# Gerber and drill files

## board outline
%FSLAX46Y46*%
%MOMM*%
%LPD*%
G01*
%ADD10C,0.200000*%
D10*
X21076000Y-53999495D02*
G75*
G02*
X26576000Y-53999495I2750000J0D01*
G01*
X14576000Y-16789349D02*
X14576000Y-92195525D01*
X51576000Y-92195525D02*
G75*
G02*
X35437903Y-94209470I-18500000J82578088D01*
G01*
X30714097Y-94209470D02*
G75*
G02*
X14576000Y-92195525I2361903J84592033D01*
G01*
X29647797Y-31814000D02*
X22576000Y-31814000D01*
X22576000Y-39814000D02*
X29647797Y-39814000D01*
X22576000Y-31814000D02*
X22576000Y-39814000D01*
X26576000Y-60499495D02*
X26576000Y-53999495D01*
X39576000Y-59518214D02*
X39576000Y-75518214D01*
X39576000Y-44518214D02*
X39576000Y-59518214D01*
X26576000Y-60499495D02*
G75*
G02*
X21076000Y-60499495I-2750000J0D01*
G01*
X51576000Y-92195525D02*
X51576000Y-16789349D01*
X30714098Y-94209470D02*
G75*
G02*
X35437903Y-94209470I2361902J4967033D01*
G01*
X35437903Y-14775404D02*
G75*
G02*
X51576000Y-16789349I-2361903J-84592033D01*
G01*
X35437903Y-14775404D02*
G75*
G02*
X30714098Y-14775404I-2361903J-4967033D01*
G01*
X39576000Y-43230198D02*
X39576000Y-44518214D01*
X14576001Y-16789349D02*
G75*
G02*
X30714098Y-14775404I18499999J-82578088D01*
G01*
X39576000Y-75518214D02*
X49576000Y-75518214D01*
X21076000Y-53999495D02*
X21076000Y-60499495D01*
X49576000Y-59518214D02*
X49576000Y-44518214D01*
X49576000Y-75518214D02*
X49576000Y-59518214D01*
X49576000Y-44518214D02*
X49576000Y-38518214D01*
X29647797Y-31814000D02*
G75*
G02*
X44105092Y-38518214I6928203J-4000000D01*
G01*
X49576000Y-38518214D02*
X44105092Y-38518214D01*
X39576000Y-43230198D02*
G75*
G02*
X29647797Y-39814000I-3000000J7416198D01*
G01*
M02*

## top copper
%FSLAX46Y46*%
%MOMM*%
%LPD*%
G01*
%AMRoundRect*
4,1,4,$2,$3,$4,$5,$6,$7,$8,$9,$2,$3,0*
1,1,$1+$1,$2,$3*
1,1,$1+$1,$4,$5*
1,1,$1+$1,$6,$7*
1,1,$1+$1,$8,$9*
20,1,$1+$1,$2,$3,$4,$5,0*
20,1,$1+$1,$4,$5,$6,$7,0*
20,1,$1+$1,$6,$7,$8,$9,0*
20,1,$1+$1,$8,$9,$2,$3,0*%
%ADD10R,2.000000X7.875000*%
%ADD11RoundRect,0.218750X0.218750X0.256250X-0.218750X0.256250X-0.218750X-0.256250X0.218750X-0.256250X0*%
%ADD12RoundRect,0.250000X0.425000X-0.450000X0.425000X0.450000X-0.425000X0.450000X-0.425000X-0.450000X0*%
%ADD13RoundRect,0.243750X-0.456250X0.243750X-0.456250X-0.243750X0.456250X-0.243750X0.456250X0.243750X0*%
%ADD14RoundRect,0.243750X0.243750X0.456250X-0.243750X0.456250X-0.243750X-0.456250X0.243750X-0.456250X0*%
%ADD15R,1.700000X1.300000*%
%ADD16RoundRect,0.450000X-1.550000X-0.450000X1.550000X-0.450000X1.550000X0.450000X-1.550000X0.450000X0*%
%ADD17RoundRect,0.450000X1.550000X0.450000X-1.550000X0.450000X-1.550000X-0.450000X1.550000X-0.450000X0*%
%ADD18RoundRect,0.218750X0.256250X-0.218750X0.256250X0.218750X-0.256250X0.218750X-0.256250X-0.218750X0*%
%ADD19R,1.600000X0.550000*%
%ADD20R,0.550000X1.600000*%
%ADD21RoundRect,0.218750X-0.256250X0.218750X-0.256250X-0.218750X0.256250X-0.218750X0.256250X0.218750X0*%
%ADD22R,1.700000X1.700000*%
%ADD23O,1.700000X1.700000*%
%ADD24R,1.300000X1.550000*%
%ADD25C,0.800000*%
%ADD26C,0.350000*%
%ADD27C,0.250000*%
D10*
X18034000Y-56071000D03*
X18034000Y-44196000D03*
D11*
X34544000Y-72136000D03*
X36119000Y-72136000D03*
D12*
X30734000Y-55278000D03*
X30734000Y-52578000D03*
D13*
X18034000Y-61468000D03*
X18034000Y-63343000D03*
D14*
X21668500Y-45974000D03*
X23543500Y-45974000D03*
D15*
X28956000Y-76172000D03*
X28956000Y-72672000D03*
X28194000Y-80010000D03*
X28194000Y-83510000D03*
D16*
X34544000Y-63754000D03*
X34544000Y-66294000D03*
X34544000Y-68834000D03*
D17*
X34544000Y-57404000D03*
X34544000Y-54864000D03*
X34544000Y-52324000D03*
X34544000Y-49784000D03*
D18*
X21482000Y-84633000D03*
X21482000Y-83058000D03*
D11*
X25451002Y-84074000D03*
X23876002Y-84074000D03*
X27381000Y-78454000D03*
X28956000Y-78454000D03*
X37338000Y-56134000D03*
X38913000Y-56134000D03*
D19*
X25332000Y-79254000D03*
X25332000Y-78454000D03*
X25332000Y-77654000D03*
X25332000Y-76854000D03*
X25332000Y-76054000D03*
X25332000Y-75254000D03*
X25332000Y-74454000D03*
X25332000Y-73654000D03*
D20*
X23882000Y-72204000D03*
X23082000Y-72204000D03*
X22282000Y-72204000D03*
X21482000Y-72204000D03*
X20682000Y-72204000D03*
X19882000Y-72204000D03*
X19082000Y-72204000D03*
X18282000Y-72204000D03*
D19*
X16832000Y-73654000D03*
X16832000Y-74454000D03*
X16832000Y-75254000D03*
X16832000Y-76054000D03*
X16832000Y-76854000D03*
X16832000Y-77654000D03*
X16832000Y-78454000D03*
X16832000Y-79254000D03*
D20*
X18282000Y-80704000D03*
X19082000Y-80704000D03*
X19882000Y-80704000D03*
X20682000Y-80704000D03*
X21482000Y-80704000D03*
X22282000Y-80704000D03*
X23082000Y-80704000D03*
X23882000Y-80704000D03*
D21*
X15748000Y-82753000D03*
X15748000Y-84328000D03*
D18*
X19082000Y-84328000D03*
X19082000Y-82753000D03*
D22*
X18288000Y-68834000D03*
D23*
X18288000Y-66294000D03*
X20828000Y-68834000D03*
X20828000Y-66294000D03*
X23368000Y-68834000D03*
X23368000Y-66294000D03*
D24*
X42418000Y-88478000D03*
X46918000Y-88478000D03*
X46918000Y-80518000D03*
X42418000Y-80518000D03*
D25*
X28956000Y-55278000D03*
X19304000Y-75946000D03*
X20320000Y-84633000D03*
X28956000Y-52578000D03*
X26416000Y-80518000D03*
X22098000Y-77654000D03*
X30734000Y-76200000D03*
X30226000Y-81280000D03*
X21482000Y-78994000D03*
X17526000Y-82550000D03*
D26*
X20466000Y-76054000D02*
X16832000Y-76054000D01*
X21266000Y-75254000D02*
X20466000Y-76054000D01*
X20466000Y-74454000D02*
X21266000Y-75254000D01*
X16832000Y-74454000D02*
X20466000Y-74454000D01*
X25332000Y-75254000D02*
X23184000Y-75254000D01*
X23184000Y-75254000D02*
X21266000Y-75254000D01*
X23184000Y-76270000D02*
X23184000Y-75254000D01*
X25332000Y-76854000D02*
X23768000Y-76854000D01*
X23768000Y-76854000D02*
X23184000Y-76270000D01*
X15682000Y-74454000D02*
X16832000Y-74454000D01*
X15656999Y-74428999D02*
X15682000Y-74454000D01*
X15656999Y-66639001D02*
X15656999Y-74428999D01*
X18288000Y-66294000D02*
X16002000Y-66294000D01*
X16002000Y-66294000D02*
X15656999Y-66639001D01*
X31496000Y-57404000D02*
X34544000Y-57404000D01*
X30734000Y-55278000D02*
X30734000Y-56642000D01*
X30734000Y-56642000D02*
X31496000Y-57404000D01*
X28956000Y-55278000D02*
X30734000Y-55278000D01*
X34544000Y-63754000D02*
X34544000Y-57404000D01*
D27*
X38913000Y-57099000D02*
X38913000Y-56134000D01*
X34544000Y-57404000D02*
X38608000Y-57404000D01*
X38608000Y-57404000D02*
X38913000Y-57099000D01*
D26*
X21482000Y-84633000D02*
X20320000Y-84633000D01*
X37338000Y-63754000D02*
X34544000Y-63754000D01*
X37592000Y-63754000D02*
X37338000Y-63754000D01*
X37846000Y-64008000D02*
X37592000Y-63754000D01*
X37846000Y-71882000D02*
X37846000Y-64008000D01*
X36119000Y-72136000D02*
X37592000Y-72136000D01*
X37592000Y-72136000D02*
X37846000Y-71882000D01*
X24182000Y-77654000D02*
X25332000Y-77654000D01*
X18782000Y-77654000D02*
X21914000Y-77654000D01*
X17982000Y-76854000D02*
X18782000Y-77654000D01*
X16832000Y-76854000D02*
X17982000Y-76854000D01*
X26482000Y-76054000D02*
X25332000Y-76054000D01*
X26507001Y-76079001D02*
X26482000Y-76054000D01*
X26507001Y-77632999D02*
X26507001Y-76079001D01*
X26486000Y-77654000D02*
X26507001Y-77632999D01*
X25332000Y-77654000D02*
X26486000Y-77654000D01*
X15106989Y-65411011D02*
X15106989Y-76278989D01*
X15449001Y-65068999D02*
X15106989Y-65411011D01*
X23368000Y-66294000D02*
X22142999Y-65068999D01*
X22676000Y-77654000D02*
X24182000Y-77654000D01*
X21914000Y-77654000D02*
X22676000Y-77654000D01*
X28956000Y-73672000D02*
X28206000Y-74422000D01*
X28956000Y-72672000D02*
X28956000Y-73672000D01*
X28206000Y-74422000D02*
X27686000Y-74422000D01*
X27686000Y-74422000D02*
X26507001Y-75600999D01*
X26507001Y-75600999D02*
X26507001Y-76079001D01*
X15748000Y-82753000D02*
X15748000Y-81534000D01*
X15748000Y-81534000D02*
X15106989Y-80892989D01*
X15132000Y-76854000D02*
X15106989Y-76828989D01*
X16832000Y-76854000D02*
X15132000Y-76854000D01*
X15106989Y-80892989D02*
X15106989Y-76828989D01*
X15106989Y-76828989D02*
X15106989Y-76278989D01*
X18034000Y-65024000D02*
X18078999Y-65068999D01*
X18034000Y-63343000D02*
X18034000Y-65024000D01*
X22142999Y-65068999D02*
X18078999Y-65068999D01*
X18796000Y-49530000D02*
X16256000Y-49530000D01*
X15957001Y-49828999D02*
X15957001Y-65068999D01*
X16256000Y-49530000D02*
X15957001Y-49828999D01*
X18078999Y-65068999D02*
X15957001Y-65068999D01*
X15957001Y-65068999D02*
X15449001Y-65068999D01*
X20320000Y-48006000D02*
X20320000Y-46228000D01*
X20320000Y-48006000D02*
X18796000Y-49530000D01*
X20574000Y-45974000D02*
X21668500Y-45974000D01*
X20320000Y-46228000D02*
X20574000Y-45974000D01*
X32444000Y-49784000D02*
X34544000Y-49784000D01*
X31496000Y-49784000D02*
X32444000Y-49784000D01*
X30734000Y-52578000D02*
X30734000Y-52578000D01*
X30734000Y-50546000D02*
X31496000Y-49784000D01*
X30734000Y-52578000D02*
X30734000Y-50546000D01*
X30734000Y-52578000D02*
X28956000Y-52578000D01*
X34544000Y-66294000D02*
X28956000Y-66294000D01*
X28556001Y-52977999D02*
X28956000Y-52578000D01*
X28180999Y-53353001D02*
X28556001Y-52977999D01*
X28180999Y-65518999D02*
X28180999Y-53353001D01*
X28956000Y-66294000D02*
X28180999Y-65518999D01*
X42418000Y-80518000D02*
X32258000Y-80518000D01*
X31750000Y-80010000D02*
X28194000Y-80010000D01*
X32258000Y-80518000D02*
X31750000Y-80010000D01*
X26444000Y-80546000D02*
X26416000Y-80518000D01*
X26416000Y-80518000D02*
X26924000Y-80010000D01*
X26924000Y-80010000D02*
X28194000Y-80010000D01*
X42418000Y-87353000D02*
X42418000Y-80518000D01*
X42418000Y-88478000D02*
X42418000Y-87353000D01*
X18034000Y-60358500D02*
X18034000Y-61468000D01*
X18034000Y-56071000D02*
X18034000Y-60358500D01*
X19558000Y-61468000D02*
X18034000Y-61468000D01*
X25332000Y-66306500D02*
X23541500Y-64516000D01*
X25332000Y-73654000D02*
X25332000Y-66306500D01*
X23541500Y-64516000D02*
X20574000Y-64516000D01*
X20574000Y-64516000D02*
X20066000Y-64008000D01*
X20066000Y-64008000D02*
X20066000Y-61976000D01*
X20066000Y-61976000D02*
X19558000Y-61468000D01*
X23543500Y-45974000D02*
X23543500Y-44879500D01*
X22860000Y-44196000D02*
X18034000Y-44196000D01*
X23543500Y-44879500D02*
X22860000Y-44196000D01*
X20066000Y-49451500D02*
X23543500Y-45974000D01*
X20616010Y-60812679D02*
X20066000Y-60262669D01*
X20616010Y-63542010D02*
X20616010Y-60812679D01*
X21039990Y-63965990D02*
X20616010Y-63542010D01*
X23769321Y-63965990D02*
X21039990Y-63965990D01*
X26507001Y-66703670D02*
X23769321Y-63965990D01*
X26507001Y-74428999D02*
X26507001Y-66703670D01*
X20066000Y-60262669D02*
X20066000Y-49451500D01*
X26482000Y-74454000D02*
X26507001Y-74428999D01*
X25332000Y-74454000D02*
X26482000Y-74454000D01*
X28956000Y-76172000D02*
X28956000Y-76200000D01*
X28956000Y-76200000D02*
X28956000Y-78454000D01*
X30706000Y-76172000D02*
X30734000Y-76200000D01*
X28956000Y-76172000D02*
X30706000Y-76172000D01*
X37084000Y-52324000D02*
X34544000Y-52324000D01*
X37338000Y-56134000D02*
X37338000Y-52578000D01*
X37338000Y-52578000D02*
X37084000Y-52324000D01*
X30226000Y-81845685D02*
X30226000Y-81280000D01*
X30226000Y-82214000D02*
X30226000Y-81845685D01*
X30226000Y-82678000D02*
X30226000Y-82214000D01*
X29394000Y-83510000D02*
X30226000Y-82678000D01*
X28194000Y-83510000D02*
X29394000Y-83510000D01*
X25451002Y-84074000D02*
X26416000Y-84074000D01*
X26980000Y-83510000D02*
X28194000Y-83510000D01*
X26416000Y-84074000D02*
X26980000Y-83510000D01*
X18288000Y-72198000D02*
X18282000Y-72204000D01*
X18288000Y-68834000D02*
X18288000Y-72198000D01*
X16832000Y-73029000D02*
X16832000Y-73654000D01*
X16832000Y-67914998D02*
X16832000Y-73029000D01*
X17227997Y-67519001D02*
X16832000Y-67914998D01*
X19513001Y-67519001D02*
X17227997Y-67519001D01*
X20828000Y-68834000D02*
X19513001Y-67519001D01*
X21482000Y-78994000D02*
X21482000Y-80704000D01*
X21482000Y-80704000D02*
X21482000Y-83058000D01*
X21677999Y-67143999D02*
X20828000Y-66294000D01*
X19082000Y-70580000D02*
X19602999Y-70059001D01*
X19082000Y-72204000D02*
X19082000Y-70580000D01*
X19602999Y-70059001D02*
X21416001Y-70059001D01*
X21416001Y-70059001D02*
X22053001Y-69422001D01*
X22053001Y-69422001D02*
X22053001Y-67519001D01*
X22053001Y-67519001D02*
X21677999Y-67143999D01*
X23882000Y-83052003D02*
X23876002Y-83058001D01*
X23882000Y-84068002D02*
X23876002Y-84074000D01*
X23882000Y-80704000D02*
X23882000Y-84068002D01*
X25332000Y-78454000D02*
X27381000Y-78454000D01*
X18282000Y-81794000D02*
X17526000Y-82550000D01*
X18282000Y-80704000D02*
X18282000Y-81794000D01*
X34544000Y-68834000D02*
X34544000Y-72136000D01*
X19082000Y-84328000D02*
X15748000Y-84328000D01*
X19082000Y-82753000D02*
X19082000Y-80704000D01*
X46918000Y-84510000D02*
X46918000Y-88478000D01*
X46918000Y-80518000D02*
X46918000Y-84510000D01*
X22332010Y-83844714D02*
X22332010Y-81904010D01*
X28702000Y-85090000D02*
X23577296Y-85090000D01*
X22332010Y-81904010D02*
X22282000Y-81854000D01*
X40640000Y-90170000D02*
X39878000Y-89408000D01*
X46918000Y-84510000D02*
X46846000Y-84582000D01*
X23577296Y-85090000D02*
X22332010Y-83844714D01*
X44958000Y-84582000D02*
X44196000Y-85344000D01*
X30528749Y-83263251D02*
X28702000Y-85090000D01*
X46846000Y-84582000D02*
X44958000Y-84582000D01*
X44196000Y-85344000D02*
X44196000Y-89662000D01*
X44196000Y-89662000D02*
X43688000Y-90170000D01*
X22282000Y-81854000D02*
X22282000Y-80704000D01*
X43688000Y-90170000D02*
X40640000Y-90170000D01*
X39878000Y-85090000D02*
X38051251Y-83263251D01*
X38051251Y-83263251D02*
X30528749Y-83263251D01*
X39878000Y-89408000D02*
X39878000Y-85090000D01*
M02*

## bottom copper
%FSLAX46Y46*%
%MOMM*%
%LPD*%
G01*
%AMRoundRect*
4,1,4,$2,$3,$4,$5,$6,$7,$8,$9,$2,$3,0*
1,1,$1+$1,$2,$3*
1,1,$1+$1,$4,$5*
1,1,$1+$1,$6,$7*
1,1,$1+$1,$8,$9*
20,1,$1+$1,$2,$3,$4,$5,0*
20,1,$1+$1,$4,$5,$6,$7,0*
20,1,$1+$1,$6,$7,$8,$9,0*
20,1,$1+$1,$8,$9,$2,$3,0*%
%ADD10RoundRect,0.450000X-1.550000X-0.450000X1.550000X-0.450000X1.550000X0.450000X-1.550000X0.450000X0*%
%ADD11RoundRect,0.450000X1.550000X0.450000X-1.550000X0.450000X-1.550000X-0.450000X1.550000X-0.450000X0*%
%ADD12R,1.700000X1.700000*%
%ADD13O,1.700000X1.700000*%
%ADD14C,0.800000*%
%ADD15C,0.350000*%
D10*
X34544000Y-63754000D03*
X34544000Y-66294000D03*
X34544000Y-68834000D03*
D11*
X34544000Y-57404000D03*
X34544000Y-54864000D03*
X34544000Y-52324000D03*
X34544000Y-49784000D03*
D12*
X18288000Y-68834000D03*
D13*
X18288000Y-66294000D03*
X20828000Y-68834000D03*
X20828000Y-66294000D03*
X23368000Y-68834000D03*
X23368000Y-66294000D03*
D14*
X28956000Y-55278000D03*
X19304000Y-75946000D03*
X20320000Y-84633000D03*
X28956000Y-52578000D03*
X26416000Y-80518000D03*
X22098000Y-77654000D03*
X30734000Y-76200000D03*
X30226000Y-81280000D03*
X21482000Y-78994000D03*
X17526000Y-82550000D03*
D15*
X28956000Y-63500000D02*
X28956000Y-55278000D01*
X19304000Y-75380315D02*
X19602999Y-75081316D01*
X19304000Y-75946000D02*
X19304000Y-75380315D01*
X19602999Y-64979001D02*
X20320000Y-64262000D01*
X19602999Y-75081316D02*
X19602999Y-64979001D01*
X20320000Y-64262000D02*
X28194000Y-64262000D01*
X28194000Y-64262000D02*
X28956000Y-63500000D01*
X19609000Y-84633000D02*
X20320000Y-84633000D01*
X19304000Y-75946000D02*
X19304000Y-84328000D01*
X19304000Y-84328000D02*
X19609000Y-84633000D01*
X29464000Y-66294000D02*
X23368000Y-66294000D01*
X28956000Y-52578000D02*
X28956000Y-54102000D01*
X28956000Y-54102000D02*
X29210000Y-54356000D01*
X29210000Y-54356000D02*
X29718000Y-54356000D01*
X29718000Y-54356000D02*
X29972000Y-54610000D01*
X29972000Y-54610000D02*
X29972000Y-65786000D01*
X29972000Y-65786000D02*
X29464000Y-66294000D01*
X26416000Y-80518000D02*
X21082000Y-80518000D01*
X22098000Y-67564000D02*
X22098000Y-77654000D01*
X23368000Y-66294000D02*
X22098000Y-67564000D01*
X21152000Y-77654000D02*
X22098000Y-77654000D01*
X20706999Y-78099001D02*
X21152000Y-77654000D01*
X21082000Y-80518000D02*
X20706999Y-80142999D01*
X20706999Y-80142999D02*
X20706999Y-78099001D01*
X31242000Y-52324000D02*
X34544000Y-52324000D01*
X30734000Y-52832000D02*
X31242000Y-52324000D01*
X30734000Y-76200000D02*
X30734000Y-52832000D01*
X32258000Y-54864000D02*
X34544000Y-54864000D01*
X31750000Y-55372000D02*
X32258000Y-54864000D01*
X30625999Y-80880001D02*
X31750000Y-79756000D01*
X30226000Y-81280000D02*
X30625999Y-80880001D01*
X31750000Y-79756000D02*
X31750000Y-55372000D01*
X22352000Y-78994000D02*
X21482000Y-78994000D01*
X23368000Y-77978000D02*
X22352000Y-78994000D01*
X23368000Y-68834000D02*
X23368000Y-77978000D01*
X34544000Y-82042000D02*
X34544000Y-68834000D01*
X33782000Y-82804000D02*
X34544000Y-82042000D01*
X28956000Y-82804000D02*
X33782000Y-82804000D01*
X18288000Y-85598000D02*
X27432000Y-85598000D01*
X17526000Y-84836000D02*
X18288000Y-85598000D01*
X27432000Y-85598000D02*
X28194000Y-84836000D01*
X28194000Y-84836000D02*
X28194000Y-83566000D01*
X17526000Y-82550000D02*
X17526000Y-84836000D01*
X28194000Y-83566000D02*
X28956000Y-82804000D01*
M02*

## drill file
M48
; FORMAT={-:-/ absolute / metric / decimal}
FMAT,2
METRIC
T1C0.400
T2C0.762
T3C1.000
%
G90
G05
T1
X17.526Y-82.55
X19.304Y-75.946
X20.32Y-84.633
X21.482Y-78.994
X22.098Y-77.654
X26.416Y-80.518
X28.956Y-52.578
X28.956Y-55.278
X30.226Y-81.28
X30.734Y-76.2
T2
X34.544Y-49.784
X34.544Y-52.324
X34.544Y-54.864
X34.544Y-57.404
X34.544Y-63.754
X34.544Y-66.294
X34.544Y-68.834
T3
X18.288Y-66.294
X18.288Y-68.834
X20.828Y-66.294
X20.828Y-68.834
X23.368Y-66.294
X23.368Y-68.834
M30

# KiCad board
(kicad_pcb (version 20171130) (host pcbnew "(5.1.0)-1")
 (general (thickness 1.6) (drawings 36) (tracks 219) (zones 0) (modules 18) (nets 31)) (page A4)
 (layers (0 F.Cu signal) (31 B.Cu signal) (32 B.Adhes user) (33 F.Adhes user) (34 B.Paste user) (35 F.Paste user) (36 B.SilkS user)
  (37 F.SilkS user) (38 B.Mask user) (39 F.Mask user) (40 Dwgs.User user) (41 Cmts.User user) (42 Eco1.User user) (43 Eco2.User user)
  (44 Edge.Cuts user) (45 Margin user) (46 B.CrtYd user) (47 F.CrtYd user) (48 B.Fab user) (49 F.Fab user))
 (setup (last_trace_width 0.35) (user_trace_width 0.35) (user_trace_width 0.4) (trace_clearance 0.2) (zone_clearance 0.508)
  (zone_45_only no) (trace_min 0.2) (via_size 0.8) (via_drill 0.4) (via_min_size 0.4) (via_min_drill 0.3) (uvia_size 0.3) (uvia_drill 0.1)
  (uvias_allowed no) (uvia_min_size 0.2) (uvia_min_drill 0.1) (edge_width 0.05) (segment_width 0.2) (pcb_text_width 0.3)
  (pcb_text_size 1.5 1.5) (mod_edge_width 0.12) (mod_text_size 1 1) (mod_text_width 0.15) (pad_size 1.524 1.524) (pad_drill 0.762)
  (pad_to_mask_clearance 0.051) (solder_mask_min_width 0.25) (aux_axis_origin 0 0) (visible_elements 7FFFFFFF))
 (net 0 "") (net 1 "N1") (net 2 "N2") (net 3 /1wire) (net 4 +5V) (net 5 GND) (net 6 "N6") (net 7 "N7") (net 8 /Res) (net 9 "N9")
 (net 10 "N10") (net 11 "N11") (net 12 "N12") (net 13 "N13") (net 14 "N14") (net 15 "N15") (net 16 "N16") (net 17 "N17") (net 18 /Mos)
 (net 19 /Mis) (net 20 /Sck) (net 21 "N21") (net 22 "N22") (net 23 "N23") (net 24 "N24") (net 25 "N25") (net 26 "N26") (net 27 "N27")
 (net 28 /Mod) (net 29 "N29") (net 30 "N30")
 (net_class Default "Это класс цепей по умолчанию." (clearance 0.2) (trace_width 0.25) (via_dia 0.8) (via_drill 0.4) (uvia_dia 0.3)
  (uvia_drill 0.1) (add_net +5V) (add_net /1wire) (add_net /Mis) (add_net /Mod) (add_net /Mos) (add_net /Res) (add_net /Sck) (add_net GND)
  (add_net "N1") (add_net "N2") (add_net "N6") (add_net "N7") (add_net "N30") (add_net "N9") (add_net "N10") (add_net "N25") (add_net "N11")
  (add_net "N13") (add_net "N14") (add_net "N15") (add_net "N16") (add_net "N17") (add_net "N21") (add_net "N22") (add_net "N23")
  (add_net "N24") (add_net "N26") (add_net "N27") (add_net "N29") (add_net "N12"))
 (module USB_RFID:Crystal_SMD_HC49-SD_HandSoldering (layer F.Cu) (at 18.034 50.1335 90)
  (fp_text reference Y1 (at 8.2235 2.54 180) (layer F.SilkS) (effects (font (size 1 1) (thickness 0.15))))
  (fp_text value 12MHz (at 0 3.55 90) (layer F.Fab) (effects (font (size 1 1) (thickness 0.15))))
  (pad 1 smd rect (at -5.9375 0 90) (size 7.875 2) (layers F.Cu F.Paste F.Mask) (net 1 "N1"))
  (pad 2 smd rect (at 5.9375 0 90) (size 7.875 2) (layers F.Cu F.Paste F.Mask) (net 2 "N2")))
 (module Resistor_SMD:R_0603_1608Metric (layer F.Cu) (at 35.3315 72.136 180)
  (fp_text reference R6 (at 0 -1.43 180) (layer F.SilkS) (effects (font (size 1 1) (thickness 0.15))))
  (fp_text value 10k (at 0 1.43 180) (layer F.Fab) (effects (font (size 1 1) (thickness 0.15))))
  (pad 2 smd roundrect (at 0.7875 0 180) (size 0.875 0.95) (layers F.Cu F.Paste F.Mask) (roundrect_rratio 0.25) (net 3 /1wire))
  (pad 1 smd roundrect (at -0.7875 0 180) (size 0.875 0.95) (layers F.Cu F.Paste F.Mask) (roundrect_rratio 0.25) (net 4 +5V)))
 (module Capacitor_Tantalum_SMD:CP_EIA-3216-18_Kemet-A (layer F.Cu) (at 30.734 53.928 90)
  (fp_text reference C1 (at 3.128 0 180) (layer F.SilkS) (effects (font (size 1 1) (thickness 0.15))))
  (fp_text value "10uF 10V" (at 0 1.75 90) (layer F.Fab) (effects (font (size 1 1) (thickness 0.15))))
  (pad 1 smd roundrect (at -1.35 0 90) (size 1.4 1.35) (layers F.Cu F.Paste F.Mask) (roundrect_rratio 0.185185) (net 4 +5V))
  (pad 2 smd roundrect (at 1.35 0 90) (size 1.4 1.35) (layers F.Cu F.Paste F.Mask) (roundrect_rratio 0.185185) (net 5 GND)))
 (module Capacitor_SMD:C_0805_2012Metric (layer F.Cu) (at 18.034 62.4055 270)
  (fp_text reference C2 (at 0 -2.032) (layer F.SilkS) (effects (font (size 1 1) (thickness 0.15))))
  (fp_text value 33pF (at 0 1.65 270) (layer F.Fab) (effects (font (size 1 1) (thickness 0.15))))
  (pad 1 smd roundrect (at -0.9375 0 270) (size 0.975 1.4) (layers F.Cu F.Paste F.Mask) (roundrect_rratio 0.25) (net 1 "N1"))
  (pad 2 smd roundrect (at 0.9375 0 270) (size 0.975 1.4) (layers F.Cu F.Paste F.Mask) (roundrect_rratio 0.25) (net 5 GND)))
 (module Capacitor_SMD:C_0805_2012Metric (layer F.Cu) (at 22.606 45.974 180)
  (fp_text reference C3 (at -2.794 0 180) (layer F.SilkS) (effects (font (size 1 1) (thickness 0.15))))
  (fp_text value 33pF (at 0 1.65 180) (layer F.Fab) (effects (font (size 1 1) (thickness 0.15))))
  (pad 2 smd roundrect (at 0.9375 0 180) (size 0.975 1.4) (layers F.Cu F.Paste F.Mask) (roundrect_rratio 0.25) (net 5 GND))
  (pad 1 smd roundrect (at -0.9375 0 180) (size 0.975 1.4) (layers F.Cu F.Paste F.Mask) (roundrect_rratio 0.25) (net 2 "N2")))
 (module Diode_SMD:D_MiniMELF (layer F.Cu) (at 28.956 74.422 90)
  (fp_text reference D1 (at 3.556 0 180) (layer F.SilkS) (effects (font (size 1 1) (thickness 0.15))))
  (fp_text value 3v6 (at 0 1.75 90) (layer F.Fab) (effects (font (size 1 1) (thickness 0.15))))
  (pad 1 smd rect (at -1.75 0 90) (size 1.3 1.7) (layers F.Cu F.Paste F.Mask) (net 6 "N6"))
  (pad 2 smd rect (at 1.75 0 90) (size 1.3 1.7) (layers F.Cu F.Paste F.Mask) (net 5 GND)))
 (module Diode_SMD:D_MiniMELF (layer F.Cu) (at 28.194 81.76 90)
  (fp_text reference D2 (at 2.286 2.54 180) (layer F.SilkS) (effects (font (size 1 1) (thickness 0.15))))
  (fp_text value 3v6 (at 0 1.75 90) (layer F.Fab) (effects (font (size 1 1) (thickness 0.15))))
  (pad 2 smd rect (at 1.75 0 90) (size 1.3 1.7) (layers F.Cu F.Paste F.Mask) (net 5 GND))
  (pad 1 smd rect (at -1.75 0 90) (size 1.3 1.7) (layers F.Cu F.Paste F.Mask) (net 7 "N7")))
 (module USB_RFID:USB (layer F.Cu) (at 34.544 61.214)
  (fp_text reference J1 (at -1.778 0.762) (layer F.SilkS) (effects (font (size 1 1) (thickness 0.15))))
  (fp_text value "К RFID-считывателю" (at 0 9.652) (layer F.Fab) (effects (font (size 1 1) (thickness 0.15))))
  (pad 1 thru_hole roundrect (at 0 2.54) (size 4 1.8) (drill 0.762) (layers *.Cu *.Mask) (roundrect_rratio 0.25) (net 4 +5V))
  (pad 2 thru_hole roundrect (at 0 5.08) (size 4 1.8) (drill 0.762) (layers *.Cu *.Mask) (roundrect_rratio 0.25) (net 5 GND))
  (pad 3 thru_hole roundrect (at 0 7.62) (size 4 1.8) (drill 0.762) (layers *.Cu *.Mask) (roundrect_rratio 0.25) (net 3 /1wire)))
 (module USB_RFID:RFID (layer F.Cu) (at 34.544 59.944 180)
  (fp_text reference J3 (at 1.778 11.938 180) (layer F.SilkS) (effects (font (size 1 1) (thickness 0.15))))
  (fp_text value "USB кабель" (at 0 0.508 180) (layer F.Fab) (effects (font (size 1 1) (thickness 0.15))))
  (pad 1 thru_hole roundrect (at 0 2.54 180) (size 4 1.8) (drill 0.762) (layers *.Cu *.Mask) (roundrect_rratio 0.25) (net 4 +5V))
  (pad 2 thru_hole roundrect (at 0 5.08 180) (size 4 1.8) (drill 0.762) (layers *.Cu *.Mask) (roundrect_rratio 0.25) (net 7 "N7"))
  (pad 3 thru_hole roundrect (at 0 7.62 180) (size 4 1.8) (drill 0.762) (layers *.Cu *.Mask) (roundrect_rratio 0.25) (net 6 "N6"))
  (pad 4 thru_hole roundrect (at 0 10.16 180) (size 4 1.8) (drill 0.762) (layers *.Cu *.Mask) (roundrect_rratio 0.25) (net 5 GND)))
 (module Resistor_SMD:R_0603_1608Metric (layer F.Cu) (at 21.482 83.8455 90)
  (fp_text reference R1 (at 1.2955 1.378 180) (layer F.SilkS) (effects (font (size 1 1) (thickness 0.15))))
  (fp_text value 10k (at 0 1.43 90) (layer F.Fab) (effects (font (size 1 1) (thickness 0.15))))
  (pad 1 smd roundrect (at -0.7875 0 90) (size 0.875 0.95) (layers F.Cu F.Paste F.Mask) (roundrect_rratio 0.25) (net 4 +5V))
  (pad 2 smd roundrect (at 0.7875 0 90) (size 0.875 0.95) (layers F.Cu F.Paste F.Mask) (roundrect_rratio 0.25) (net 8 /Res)))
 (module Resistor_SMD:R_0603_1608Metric (layer F.Cu) (at 24.663502 84.074 180)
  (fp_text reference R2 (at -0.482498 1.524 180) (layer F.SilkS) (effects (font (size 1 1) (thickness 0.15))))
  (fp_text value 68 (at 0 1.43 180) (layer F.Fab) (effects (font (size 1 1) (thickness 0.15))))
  (pad 1 smd roundrect (at -0.7875 0 180) (size 0.875 0.95) (layers F.Cu F.Paste F.Mask) (roundrect_rratio 0.25) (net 7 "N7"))
  (pad 2 smd roundrect (at 0.7875 0 180) (size 0.875 0.95) (layers F.Cu F.Paste F.Mask) (roundrect_rratio 0.25) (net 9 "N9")))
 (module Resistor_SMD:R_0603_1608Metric (layer F.Cu) (at 28.1685 78.454 180)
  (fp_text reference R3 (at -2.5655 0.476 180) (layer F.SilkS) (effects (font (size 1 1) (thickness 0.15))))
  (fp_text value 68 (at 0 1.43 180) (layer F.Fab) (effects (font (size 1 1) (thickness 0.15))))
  (pad 2 smd roundrect (at 0.7875 0 180) (size 0.875 0.95) (layers F.Cu F.Paste F.Mask) (roundrect_rratio 0.25) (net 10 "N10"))
  (pad 1 smd roundrect (at -0.7875 0 180) (size 0.875 0.95) (layers F.Cu F.Paste F.Mask) (roundrect_rratio 0.25) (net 6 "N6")))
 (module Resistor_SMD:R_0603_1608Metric (layer F.Cu) (at 38.1255 56.134 180)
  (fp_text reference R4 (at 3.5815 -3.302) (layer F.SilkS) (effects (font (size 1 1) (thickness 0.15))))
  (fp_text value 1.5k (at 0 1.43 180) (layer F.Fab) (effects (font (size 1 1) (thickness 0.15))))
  (pad 2 smd roundrect (at 0.7875 0 180) (size 0.875 0.95) (layers F.Cu F.Paste F.Mask) (roundrect_rratio 0.25) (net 6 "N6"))
  (pad 1 smd roundrect (at -0.7875 0 180) (size 0.875 0.95) (layers F.Cu F.Paste F.Mask) (roundrect_rratio 0.25) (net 4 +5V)))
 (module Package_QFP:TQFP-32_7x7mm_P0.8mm (layer F.Cu) (at 21.082 76.454 180)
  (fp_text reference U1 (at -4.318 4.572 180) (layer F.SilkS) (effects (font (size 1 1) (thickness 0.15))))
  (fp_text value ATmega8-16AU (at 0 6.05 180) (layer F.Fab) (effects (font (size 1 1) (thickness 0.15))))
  (pad 1 smd rect (at -4.25 -2.8 180) (size 1.6 0.55) (layers F.Cu F.Paste F.Mask) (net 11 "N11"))
  (pad 2 smd rect (at -4.25 -2 180) (size 1.6 0.55) (layers F.Cu F.Paste F.Mask) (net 10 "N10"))
  (pad 3 smd rect (at -4.25 -1.2 180) (size 1.6 0.55) (layers F.Cu F.Paste F.Mask) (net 5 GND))
  (pad 4 smd rect (at -4.25 -0.4 180) (size 1.6 0.55) (layers F.Cu F.Paste F.Mask) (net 4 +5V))
  (pad 5 smd rect (at -4.25 0.4 180) (size 1.6 0.55) (layers F.Cu F.Paste F.Mask) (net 5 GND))
  (pad 6 smd rect (at -4.25 1.2 180) (size 1.6 0.55) (layers F.Cu F.Paste F.Mask) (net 4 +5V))
  (pad 7 smd rect (at -4.25 2 180) (size 1.6 0.55) (layers F.Cu F.Paste F.Mask) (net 2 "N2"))
  (pad 8 smd rect (at -4.25 2.8 180) (size 1.6 0.55) (layers F.Cu F.Paste F.Mask) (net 1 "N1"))
  (pad 9 smd rect (at -2.8 4.25 270) (size 1.6 0.55) (layers F.Cu F.Paste F.Mask) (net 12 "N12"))
  (pad 10 smd rect (at -2 4.25 270) (size 1.6 0.55) (layers F.Cu F.Paste F.Mask) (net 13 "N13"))
  (pad 11 smd rect (at -1.2 4.25 270) (size 1.6 0.55) (layers F.Cu F.Paste F.Mask) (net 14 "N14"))
  (pad 12 smd rect (at -0.4 4.25 270) (size 1.6 0.55) (layers F.Cu F.Paste F.Mask) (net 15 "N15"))
  (pad 13 smd rect (at 0.4 4.25 270) (size 1.6 0.55) (layers F.Cu F.Paste F.Mask) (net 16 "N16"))
  (pad 14 smd rect (at 1.2 4.25 270) (size 1.6 0.55) (layers F.Cu F.Paste F.Mask) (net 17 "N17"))
  (pad 15 smd rect (at 2 4.25 270) (size 1.6 0.55) (layers F.Cu F.Paste F.Mask) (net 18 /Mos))
  (pad 16 smd rect (at 2.8 4.25 270) (size 1.6 0.55) (layers F.Cu F.Paste F.Mask) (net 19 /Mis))
  (pad 17 smd rect (at 4.25 2.8 180) (size 1.6 0.55) (layers F.Cu F.Paste F.Mask) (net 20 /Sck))
  (pad 18 smd rect (at 4.25 2 180) (size 1.6 0.55) (layers F.Cu F.Paste F.Mask) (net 4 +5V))
  (pad 19 smd rect (at 4.25 1.2 180) (size 1.6 0.55) (layers F.Cu F.Paste F.Mask) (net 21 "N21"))
  (pad 20 smd rect (at 4.25 0.4 180) (size 1.6 0.55) (layers F.Cu F.Paste F.Mask) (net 4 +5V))
  (pad 21 smd rect (at 4.25 -0.4 180) (size 1.6 0.55) (layers F.Cu F.Paste F.Mask) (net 5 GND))
  (pad 22 smd rect (at 4.25 -1.2 180) (size 1.6 0.55) (layers F.Cu F.Paste F.Mask) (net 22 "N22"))
  (pad 23 smd rect (at 4.25 -2 180) (size 1.6 0.55) (layers F.Cu F.Paste F.Mask) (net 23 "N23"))
  (pad 24 smd rect (at 4.25 -2.8 180) (size 1.6 0.55) (layers F.Cu F.Paste F.Mask) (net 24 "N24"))
  (pad 25 smd rect (at 2.8 -4.25 270) (size 1.6 0.55) (layers F.Cu F.Paste F.Mask) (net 3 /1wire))
  (pad 26 smd rect (at 2 -4.25 270) (size 1.6 0.55) (layers F.Cu F.Paste F.Mask) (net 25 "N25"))
  (pad 27 smd rect (at 1.2 -4.25 270) (size 1.6 0.55) (layers F.Cu F.Paste F.Mask) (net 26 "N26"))
  (pad 28 smd rect (at 0.4 -4.25 270) (size 1.6 0.55) (layers F.Cu F.Paste F.Mask) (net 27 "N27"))
  (pad 29 smd rect (at -0.4 -4.25 270) (size 1.6 0.55) (layers F.Cu F.Paste F.Mask) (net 8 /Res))
  (pad 30 smd rect (at -1.2 -4.25 270) (size 1.6 0.55) (layers F.Cu F.Paste F.Mask) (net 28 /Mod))
  (pad 31 smd rect (at -2 -4.25 270) (size 1.6 0.55) (layers F.Cu F.Paste F.Mask) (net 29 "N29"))
  (pad 32 smd rect (at -2.8 -4.25 270) (size 1.6 0.55) (layers F.Cu F.Paste F.Mask) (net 9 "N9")))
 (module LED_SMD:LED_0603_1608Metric (layer F.Cu) (at 15.748 83.5405 270)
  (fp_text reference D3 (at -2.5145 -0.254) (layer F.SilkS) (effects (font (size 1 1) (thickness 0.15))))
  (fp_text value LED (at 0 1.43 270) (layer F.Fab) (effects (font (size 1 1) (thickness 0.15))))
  (pad 1 smd roundrect (at -0.7875 0 270) (size 0.875 0.95) (layers F.Cu F.Paste F.Mask) (roundrect_rratio 0.25) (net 5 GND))
  (pad 2 smd roundrect (at 0.7875 0 270) (size 0.875 0.95) (layers F.Cu F.Paste F.Mask) (roundrect_rratio 0.25) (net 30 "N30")))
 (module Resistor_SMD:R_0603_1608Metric (layer F.Cu) (at 19.082 83.5405 90)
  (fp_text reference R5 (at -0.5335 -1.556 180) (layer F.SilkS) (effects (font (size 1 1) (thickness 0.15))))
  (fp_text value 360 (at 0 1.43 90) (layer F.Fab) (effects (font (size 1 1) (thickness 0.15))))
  (pad 1 smd roundrect (at -0.7875 0 90) (size 0.875 0.95) (layers F.Cu F.Paste F.Mask) (roundrect_rratio 0.25) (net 30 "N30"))
  (pad 2 smd roundrect (at 0.7875 0 90) (size 0.875 0.95) (layers F.Cu F.Paste F.Mask) (roundrect_rratio 0.25) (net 25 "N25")))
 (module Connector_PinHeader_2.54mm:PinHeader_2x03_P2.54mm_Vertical (layer F.Cu) (at 18.288 68.834 90)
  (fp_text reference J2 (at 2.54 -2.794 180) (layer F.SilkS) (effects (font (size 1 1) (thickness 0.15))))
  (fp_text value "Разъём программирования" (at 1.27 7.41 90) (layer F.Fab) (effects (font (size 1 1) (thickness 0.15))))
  (pad 1 thru_hole rect (at 0 0 90) (size 1.7 1.7) (drill 1) (layers *.Cu *.Mask) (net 19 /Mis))
  (pad 6 thru_hole oval (at 2.54 0 90) (size 1.7 1.7) (drill 1) (layers *.Cu *.Mask) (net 4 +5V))
  (pad 2 thru_hole oval (at 0 2.54 90) (size 1.7 1.7) (drill 1) (layers *.Cu *.Mask) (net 20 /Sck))
  (pad 5 thru_hole oval (at 2.54 2.54 90) (size 1.7 1.7) (drill 1) (layers *.Cu *.Mask) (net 18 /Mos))
  (pad 3 thru_hole oval (at 0 5.08 90) (size 1.7 1.7) (drill 1) (layers *.Cu *.Mask) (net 8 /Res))
  (pad 4 thru_hole oval (at 2.54 5.08 90) (size 1.7 1.7) (drill 1) (layers *.Cu *.Mask) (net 5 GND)))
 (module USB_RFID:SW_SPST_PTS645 (layer F.Cu) (at 44.668 84.498 270)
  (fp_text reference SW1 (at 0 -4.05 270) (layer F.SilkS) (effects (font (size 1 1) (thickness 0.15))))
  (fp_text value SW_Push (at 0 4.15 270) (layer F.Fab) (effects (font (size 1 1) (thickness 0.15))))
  (pad 2 smd rect (at 3.98 2.25 270) (size 1.55 1.3) (layers F.Cu F.Paste F.Mask) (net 5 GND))
  (pad 1 smd rect (at 3.98 -2.25 270) (size 1.55 1.3) (layers F.Cu F.Paste F.Mask) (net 28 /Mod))
  (pad 1 smd rect (at -3.98 -2.25 270) (size 1.55 1.3) (layers F.Cu F.Paste F.Mask) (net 28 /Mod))
  (pad 2 smd rect (at -3.98 2.25 270) (size 1.55 1.3) (layers F.Cu F.Paste F.Mask) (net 5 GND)))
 (gr_arc (start 23.826 53.999495) (end 26.576 53.999495) (angle -180) (layer Edge.Cuts) (width 0.2))
 (gr_line (start 14.576 16.789349) (end 14.576 92.195525) (layer Edge.Cuts) (width 0.2))
 (gr_arc (start 33.076 9.617437) (end 35.437903 94.20947) (angle -11.02814845) (layer Edge.Cuts) (width 0.2))
 (gr_arc (start 33.076 9.617437) (end 14.576 92.195525) (angle -11.02814845) (layer Edge.Cuts) (width 0.2))
 (gr_line (start 29.647797 31.814) (end 22.576 31.814) (layer Edge.Cuts) (width 0.2))
 (gr_line (start 22.576 39.814) (end 29.647797 39.814) (layer Edge.Cuts) (width 0.2))
 (gr_line (start 22.576 31.814) (end 22.576 39.814) (layer Edge.Cuts) (width 0.2))
 (gr_line (start 26.576 60.499495) (end 26.576 53.999495) (layer Edge.Cuts) (width 0.2))
 (gr_line (start 39.576 59.518214) (end 39.576 75.518214) (layer Edge.Cuts) (width 0.2))
 (gr_line (start 39.576 44.518214) (end 39.576 59.518214) (layer Edge.Cuts) (width 0.2))
 (gr_arc (start 23.826 60.499495) (end 21.076 60.499495) (angle -180) (layer Edge.Cuts) (width 0.2))
 (gr_line (start 51.576 92.195525) (end 51.576 16.789349) (layer Edge.Cuts) (width 0.2))
 (gr_arc (start 33.076 89.242437) (end 35.437903 94.20947) (angle -309.1363505) (layer Edge.Cuts) (width 0.2))
 (gr_arc (start 33.076 99.367437) (end 51.576 16.789349) (angle -11.02814845) (layer Edge.Cuts) (width 0.2))
 (gr_arc (start 33.076 19.742437) (end 30.714098 14.775404) (angle -309.1363506) (layer Edge.Cuts) (width 0.2))
 (gr_line (start 39.576 43.230198) (end 39.576 44.518214) (layer Edge.Cuts) (width 0.2))
 (gr_arc (start 33.076 99.367437) (end 30.714098 14.775404) (angle -11.02814845) (layer Edge.Cuts) (width 0.2))
 (gr_line (start 39.576 75.518214) (end 49.576 75.518214) (layer Edge.Cuts) (width 0.2))
 (gr_line (start 21.076 53.999495) (end 21.076 60.499495) (layer Edge.Cuts) (width 0.2))
 (gr_line (start 49.576 59.518214) (end 49.576 44.518214) (layer Edge.Cuts) (width 0.2))
 (gr_line (start 49.576 75.518214) (end 49.576 59.518214) (layer Edge.Cuts) (width 0.2))
 (gr_line (start 49.576 44.518214) (end 49.576 38.518214) (layer Edge.Cuts) (width 0.2))
 (gr_arc (start 36.576 35.814) (end 44.105092 38.518214) (angle -169.7567013) (layer Edge.Cuts) (width 0.2))
 (gr_line (start 49.576 38.518214) (end 44.105092 38.518214) (layer Edge.Cuts) (width 0.2))
 (gr_arc (start 36.576 35.814) (end 29.647797 39.814) (angle -82.02431284) (layer Edge.Cuts) (width 0.2))
 (via (at 28.956 55.278) (size 0.8) (drill 0.4) (layers F.Cu B.Cu) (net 4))
 (via (at 19.304 75.946) (size 0.8) (drill 0.4) (layers F.Cu B.Cu) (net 4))
 (segment (start 20.466 76.054) (end 16.832 76.054) (width 0.35) (layer F.Cu) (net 4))
 (segment (start 21.266 75.254) (end 20.466 76.054) (width 0.35) (layer F.Cu) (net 4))
 (segment (start 20.466 74.454) (end 21.266 75.254) (width 0.35) (layer F.Cu) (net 4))
 (segment (start 16.832 74.454) (end 20.466 74.454) (width 0.35) (layer F.Cu) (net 4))
 (segment (start 25.332 75.254) (end 23.184 75.254) (width 0.35) (layer F.Cu) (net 4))
 (segment (start 23.184 75.254) (end 21.266 75.254) (width 0.35) (layer F.Cu) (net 4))
 (segment (start 23.184 76.27) (end 23.184 75.254) (width 0.35) (layer F.Cu) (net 4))
 (segment (start 25.332 76.854) (end 23.768 76.854) (width 0.35) (layer F.Cu) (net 4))
 (segment (start 23.768 76.854) (end 23.184 76.27) (width 0.35) (layer F.Cu) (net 4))
 (segment (start 15.682 74.454) (end 16.832 74.454) (width 0.35) (layer F.Cu) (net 4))
 (segment (start 15.656999 74.428999) (end 15.682 74.454) (width 0.35) (layer F.Cu) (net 4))
 (segment (start 15.656999 66.639001) (end 15.656999 74.428999) (width 0.35) (layer F.Cu) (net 4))
 (segment (start 18.288 66.294) (end 16.002 66.294) (width 0.35) (layer F.Cu) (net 4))
 (segment (start 16.002 66.294) (end 15.656999 66.639001) (width 0.35) (layer F.Cu) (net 4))
 (segment (start 31.496 57.404) (end 34.544 57.404) (width 0.35) (layer F.Cu) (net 4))
 (segment (start 30.734 55.278) (end 30.734 56.642) (width 0.35) (layer F.Cu) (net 4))
 (segment (start 30.734 56.642) (end 31.496 57.404) (width 0.35) (layer F.Cu) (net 4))
 (segment (start 28.956 55.278) (end 30.734 55.278) (width 0.35) (layer F.Cu) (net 4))
 (segment (start 28.956 63.5) (end 28.956 55.278) (width 0.35) (layer B.Cu) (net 4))
 (segment (start 19.304 75.380315) (end 19.602999 75.081316) (width 0.35) (layer B.Cu) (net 4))
 (segment (start 19.304 75.946) (end 19.304 75.380315) (width 0.35) (layer B.Cu) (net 4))
 (segment (start 19.602999 64.979001) (end 20.32 64.262) (width 0.35) (layer B.Cu) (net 4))
 (segment (start 19.602999 75.081316) (end 19.602999 64.979001) (width 0.35) (layer B.Cu) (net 4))
 (segment (start 20.32 64.262) (end 28.194 64.262) (width 0.35) (layer B.Cu) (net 4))
 (segment (start 28.194 64.262) (end 28.956 63.5) (width 0.35) (layer B.Cu) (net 4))
 (segment (start 34.544 63.754) (end 34.544 57.404) (width 0.35) (layer F.Cu) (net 4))
 (segment (start 38.913 57.099) (end 38.913 56.134) (width 0.25) (layer F.Cu) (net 4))
 (segment (start 34.544 57.404) (end 38.608 57.404) (width 0.25) (layer F.Cu) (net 4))
 (segment (start 38.608 57.404) (end 38.913 57.099) (width 0.25) (layer F.Cu) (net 4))
 (via (at 20.32 84.633) (size 0.8) (drill 0.4) (layers F.Cu B.Cu) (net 4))
 (segment (start 19.609 84.633) (end 20.32 84.633) (width 0.35) (layer B.Cu) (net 4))
 (segment (start 19.304 75.946) (end 19.304 84.328) (width 0.35) (layer B.Cu) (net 4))
 (segment (start 19.304 84.328) (end 19.609 84.633) (width 0.35) (layer B.Cu) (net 4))
 (segment (start 21.482 84.633) (end 20.32 84.633) (width 0.35) (layer F.Cu) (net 4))
 (segment (start 37.338 63.754) (end 34.544 63.754) (width 0.35) (layer F.Cu) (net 4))
 (segment (start 37.592 63.754) (end 37.338 63.754) (width 0.35) (layer F.Cu) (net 4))
 (segment (start 37.846 64.008) (end 37.592 63.754) (width 0.35) (layer F.Cu) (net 4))
 (segment (start 37.846 71.882) (end 37.846 64.008) (width 0.35) (layer F.Cu) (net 4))
 (segment (start 36.119 72.136) (end 37.592 72.136) (width 0.35) (layer F.Cu) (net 4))
 (segment (start 37.592 72.136) (end 37.846 71.882) (width 0.35) (layer F.Cu) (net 4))
 (segment (start 24.182 77.654) (end 25.332 77.654) (width 0.35) (layer F.Cu) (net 5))
 (segment (start 18.782 77.654) (end 21.914 77.654) (width 0.35) (layer F.Cu) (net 5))
 (segment (start 17.982 76.854) (end 18.782 77.654) (width 0.35) (layer F.Cu) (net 5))
 (segment (start 16.832 76.854) (end 17.982 76.854) (width 0.35) (layer F.Cu) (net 5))
 (segment (start 26.482 76.054) (end 25.332 76.054) (width 0.35) (layer F.Cu) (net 5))
 (segment (start 26.507001 76.079001) (end 26.482 76.054) (width 0.35) (layer F.Cu) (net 5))
 (segment (start 26.507001 77.632999) (end 26.507001 76.079001) (width 0.35) (layer F.Cu) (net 5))
 (segment (start 26.486 77.654) (end 26.507001 77.632999) (width 0.35) (layer F.Cu) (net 5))
 (segment (start 25.332 77.654) (end 26.486 77.654) (width 0.35) (layer F.Cu) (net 5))
 (segment (start 15.106989 65.411011) (end 15.106989 76.278989) (width 0.35) (layer F.Cu) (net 5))
 (segment (start 15.449001 65.068999) (end 15.106989 65.411011) (width 0.35) (layer F.Cu) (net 5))
 (segment (start 23.368 66.294) (end 22.142999 65.068999) (width 0.35) (layer F.Cu) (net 5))
 (segment (start 22.676 77.654) (end 24.182 77.654) (width 0.35) (layer F.Cu) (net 5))
 (segment (start 21.914 77.654) (end 22.676 77.654) (width 0.35) (layer F.Cu) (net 5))
 (segment (start 28.956 73.672) (end 28.206 74.422) (width 0.35) (layer F.Cu) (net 5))
 (segment (start 28.956 72.672) (end 28.956 73.672) (width 0.35) (layer F.Cu) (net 5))
 (segment (start 28.206 74.422) (end 27.686 74.422) (width 0.35) (layer F.Cu) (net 5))
 (segment (start 27.686 74.422) (end 26.507001 75.600999) (width 0.35) (layer F.Cu) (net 5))
 (segment (start 26.507001 75.600999) (end 26.507001 76.079001) (width 0.35) (layer F.Cu) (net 5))
 (segment (start 15.748 82.753) (end 15.748 81.534) (width 0.35) (layer F.Cu) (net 5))
 (segment (start 15.748 81.534) (end 15.106989 80.892989) (width 0.35) (layer F.Cu) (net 5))
 (segment (start 15.132 76.854) (end 15.106989 76.828989) (width 0.35) (layer F.Cu) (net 5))
 (segment (start 16.832 76.854) (end 15.132 76.854) (width 0.35) (layer F.Cu) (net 5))
 (segment (start 15.106989 80.892989) (end 15.106989 76.828989) (width 0.35) (layer F.Cu) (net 5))
 (segment (start 15.106989 76.828989) (end 15.106989 76.278989) (width 0.35) (layer F.Cu) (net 5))
 (segment (start 18.034 65.024) (end 18.078999 65.068999) (width 0.35) (layer F.Cu) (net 5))
 (segment (start 18.034 63.343) (end 18.034 65.024) (width 0.35) (layer F.Cu) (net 5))
 (segment (start 22.142999 65.068999) (end 18.078999 65.068999) (width 0.35) (layer F.Cu) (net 5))
 (segment (start 18.796 49.53) (end 16.256 49.53) (width 0.35) (layer F.Cu) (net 5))
 (segment (start 15.957001 49.828999) (end 15.957001 65.068999) (width 0.35) (layer F.Cu) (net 5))
 (segment (start 16.256 49.53) (end 15.957001 49.828999) (width 0.35) (layer F.Cu) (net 5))
 (segment (start 18.078999 65.068999) (end 15.957001 65.068999) (width 0.35) (layer F.Cu) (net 5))
 (segment (start 15.957001 65.068999) (end 15.449001 65.068999) (width 0.35) (layer F.Cu) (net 5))
 (segment (start 20.32 48.006) (end 20.32 46.228) (width 0.35) (layer F.Cu) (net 5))
 (segment (start 20.32 48.006) (end 18.796 49.53) (width 0.35) (layer F.Cu) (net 5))
 (segment (start 20.574 45.974) (end 21.6685 45.974) (width 0.35) (layer F.Cu) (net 5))
 (segment (start 20.32 46.228) (end 20.574 45.974) (width 0.35) (layer F.Cu) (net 5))
 (segment (start 32.444 49.784) (end 34.544 49.784) (width 0.35) (layer F.Cu) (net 5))
 (segment (start 31.496 49.784) (end 32.444 49.784) (width 0.35) (layer F.Cu) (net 5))
 (segment (start 30.734 52.578) (end 30.734 52.578) (width 0.35) (layer F.Cu) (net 5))
 (segment (start 30.734 50.546) (end 31.496 49.784) (width 0.35) (layer F.Cu) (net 5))
 (segment (start 30.734 52.578) (end 30.734 50.546) (width 0.35) (layer F.Cu) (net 5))
 (via (at 28.956 52.578) (size 0.8) (drill 0.4) (layers F.Cu B.Cu) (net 5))
 (segment (start 30.734 52.578) (end 28.956 52.578) (width 0.35) (layer F.Cu) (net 5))
 (segment (start 29.464 66.294) (end 23.368 66.294) (width 0.35) (layer B.Cu) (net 5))
 (segment (start 28.956 52.578) (end 28.956 54.102) (width 0.35) (layer B.Cu) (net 5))
 (segment (start 28.956 54.102) (end 29.21 54.356) (width 0.35) (layer B.Cu) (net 5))
 (segment (start 29.21 54.356) (end 29.718 54.356) (width 0.35) (layer B.Cu) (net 5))
 (segment (start 29.718 54.356) (end 29.972 54.61) (width 0.35) (layer B.Cu) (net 5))
 (segment (start 29.972 54.61) (end 29.972 65.786) (width 0.35) (layer B.Cu) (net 5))
 (segment (start 29.972 65.786) (end 29.464 66.294) (width 0.35) (layer B.Cu) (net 5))
 (segment (start 34.544 66.294) (end 28.956 66.294) (width 0.35) (layer F.Cu) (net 5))
 (segment (start 28.556001 52.977999) (end 28.956 52.578) (width 0.35) (layer F.Cu) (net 5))
 (segment (start 28.180999 53.353001) (end 28.556001 52.977999) (width 0.35) (layer F.Cu) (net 5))
 (segment (start 28.180999 65.518999) (end 28.180999 53.353001) (width 0.35) (layer F.Cu) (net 5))
 (segment (start 28.956 66.294) (end 28.180999 65.518999) (width 0.35) (layer F.Cu) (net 5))
 (segment (start 42.418 80.518) (end 32.258 80.518) (width 0.35) (layer F.Cu) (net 5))
 (segment (start 31.75 80.01) (end 28.194 80.01) (width 0.35) (layer F.Cu) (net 5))
 (segment (start 32.258 80.518) (end 31.75 80.01) (width 0.35) (layer F.Cu) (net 5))
 (segment (start 26.416 80.518) (end 21.082 80.518) (width 0.35) (layer B.Cu) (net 5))
 (segment (start 22.098 67.564) (end 22.098 77.654) (width 0.35) (layer B.Cu) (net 5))
 (segment (start 23.368 66.294) (end 22.098 67.564) (width 0.35) (layer B.Cu) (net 5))
 (segment (start 26.444 80.546) (end 26.416 80.518) (width 0.35) (layer F.Cu) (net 5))
 (segment (start 21.152 77.654) (end 22.098 77.654) (width 0.35) (layer B.Cu) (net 5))
 (segment (start 20.706999 78.099001) (end 21.152 77.654) (width 0.35) (layer B.Cu) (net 5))
 (segment (start 21.082 80.518) (end 20.706999 80.142999) (width 0.35) (layer B.Cu) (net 5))
 (segment (start 20.706999 80.142999) (end 20.706999 78.099001) (width 0.35) (layer B.Cu) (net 5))
 (via (at 26.416 80.518) (size 0.8) (drill 0.4) (layers F.Cu B.Cu) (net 5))
 (via (at 22.098 77.654) (size 0.8) (drill 0.4) (layers F.Cu B.Cu) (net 5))
 (segment (start 26.416 80.518) (end 26.924 80.01) (width 0.35) (layer F.Cu) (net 5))
 (segment (start 26.924 80.01) (end 28.194 80.01) (width 0.35) (layer F.Cu) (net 5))
 (segment (start 42.418 87.353) (end 42.418 80.518) (width 0.35) (layer F.Cu) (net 5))
 (segment (start 42.418 88.478) (end 42.418 87.353) (width 0.35) (layer F.Cu) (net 5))
 (segment (start 18.034 60.3585) (end 18.034 61.468) (width 0.35) (layer F.Cu) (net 1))
 (segment (start 18.034 56.071) (end 18.034 60.3585) (width 0.35) (layer F.Cu) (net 1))
 (segment (start 19.558 61.468) (end 18.034 61.468) (width 0.35) (layer F.Cu) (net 1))
 (segment (start 25.332 66.3065) (end 23.5415 64.516) (width 0.35) (layer F.Cu) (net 1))
 (segment (start 25.332 73.654) (end 25.332 66.3065) (width 0.35) (layer F.Cu) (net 1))
 (segment (start 23.5415 64.516) (end 20.574 64.516) (width 0.35) (layer F.Cu) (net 1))
 (segment (start 20.574 64.516) (end 20.066 64.008) (width 0.35) (layer F.Cu) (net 1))
 (segment (start 20.066 64.008) (end 20.066 61.976) (width 0.35) (layer F.Cu) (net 1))
 (segment (start 20.066 61.976) (end 19.558 61.468) (width 0.35) (layer F.Cu) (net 1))
 (segment (start 23.5435 45.974) (end 23.5435 44.8795) (width 0.35) (layer F.Cu) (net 2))
 (segment (start 22.86 44.196) (end 18.034 44.196) (width 0.35) (layer F.Cu) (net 2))
 (segment (start 23.5435 44.8795) (end 22.86 44.196) (width 0.35) (layer F.Cu) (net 2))
 (segment (start 20.066 49.4515) (end 23.5435 45.974) (width 0.35) (layer F.Cu) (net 2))
 (segment (start 20.61601 60.812679) (end 20.066 60.262669) (width 0.35) (layer F.Cu) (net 2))
 (segment (start 20.61601 63.54201) (end 20.61601 60.812679) (width 0.35) (layer F.Cu) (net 2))
 (segment (start 21.03999 63.96599) (end 20.61601 63.54201) (width 0.35) (layer F.Cu) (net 2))
 (segment (start 23.769321 63.96599) (end 21.03999 63.96599) (width 0.35) (layer F.Cu) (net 2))
 (segment (start 26.507001 66.70367) (end 23.769321 63.96599) (width 0.35) (layer F.Cu) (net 2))
 (segment (start 26.507001 74.428999) (end 26.507001 66.70367) (width 0.35) (layer F.Cu) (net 2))
 (segment (start 20.066 60.262669) (end 20.066 49.4515) (width 0.35) (layer F.Cu) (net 2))
 (segment (start 26.482 74.454) (end 26.507001 74.428999) (width 0.35) (layer F.Cu) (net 2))
 (segment (start 25.332 74.454) (end 26.482 74.454) (width 0.35) (layer F.Cu) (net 2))
 (segment (start 28.956 76.172) (end 28.956 76.2) (width 0.35) (layer F.Cu) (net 6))
 (segment (start 28.956 76.2) (end 28.956 78.454) (width 0.35) (layer F.Cu) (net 6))
 (via (at 30.734 76.2) (size 0.8) (drill 0.4) (layers F.Cu B.Cu) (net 6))
 (segment (start 30.706 76.172) (end 30.734 76.2) (width 0.35) (layer F.Cu) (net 6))
 (segment (start 28.956 76.172) (end 30.706 76.172) (width 0.35) (layer F.Cu) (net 6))
 (segment (start 31.242 52.324) (end 34.544 52.324) (width 0.35) (layer B.Cu) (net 6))
 (segment (start 30.734 52.832) (end 31.242 52.324) (width 0.35) (layer B.Cu) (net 6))
 (segment (start 30.734 76.2) (end 30.734 52.832) (width 0.35) (layer B.Cu) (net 6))
 (segment (start 37.084 52.324) (end 34.544 52.324) (width 0.35) (layer F.Cu) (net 6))
 (segment (start 37.338 56.134) (end 37.338 52.578) (width 0.35) (layer F.Cu) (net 6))
 (segment (start 37.338 52.578) (end 37.084 52.324) (width 0.35) (layer F.Cu) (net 6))
 (via (at 30.226 81.28) (size 0.8) (drill 0.4) (layers F.Cu B.Cu) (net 7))
 (segment (start 32.258 54.864) (end 34.544 54.864) (width 0.35) (layer B.Cu) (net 7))
 (segment (start 31.75 55.372) (end 32.258 54.864) (width 0.35) (layer B.Cu) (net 7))
 (segment (start 30.226 81.845685) (end 30.226 81.28) (width 0.35) (layer F.Cu) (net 7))
 (segment (start 30.226 82.214) (end 30.226 81.845685) (width 0.35) (layer F.Cu) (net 7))
 (segment (start 30.625999 80.880001) (end 31.75 79.756) (width 0.35) (layer B.Cu) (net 7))
 (segment (start 30.226 81.28) (end 30.625999 80.880001) (width 0.35) (layer B.Cu) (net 7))
 (segment (start 31.75 79.756) (end 31.75 55.372) (width 0.35) (layer B.Cu) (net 7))
 (segment (start 30.226 82.678) (end 30.226 82.214) (width 0.35) (layer F.Cu) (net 7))
 (segment (start 29.394 83.51) (end 30.226 82.678) (width 0.35) (layer F.Cu) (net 7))
 (segment (start 28.194 83.51) (end 29.394 83.51) (width 0.35) (layer F.Cu) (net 7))
 (segment (start 25.451002 84.074) (end 26.416 84.074) (width 0.35) (layer F.Cu) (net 7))
 (segment (start 26.98 83.51) (end 28.194 83.51) (width 0.35) (layer F.Cu) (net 7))
 (segment (start 26.416 84.074) (end 26.98 83.51) (width 0.35) (layer F.Cu) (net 7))
 (segment (start 18.288 72.198) (end 18.282 72.204) (width 0.35) (layer F.Cu) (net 19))
 (segment (start 18.288 68.834) (end 18.288 72.198) (width 0.35) (layer F.Cu) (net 19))
 (segment (start 16.832 73.029) (end 16.832 73.654) (width 0.35) (layer F.Cu) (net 20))
 (segment (start 16.832 67.914998) (end 16.832 73.029) (width 0.35) (layer F.Cu) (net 20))
 (segment (start 17.227997 67.519001) (end 16.832 67.914998) (width 0.35) (layer F.Cu) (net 20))
 (segment (start 19.513001 67.519001) (end 17.227997 67.519001) (width 0.35) (layer F.Cu) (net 20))
 (segment (start 20.828 68.834) (end 19.513001 67.519001) (width 0.35) (layer F.Cu) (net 20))
 (via (at 21.482 78.994) (size 0.8) (drill 0.4) (layers F.Cu B.Cu) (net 8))
 (segment (start 22.352 78.994) (end 21.482 78.994) (width 0.35) (layer B.Cu) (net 8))
 (segment (start 23.368 77.978) (end 22.352 78.994) (width 0.35) (layer B.Cu) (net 8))
 (segment (start 23.368 68.834) (end 23.368 77.978) (width 0.35) (layer B.Cu) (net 8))
 (segment (start 21.482 78.994) (end 21.482 80.704) (width 0.35) (layer F.Cu) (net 8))
 (segment (start 21.482 80.704) (end 21.482 83.058) (width 0.35) (layer F.Cu) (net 8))
 (segment (start 21.677999 67.143999) (end 20.828 66.294) (width 0.35) (layer F.Cu) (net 18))
 (segment (start 19.082 70.58) (end 19.602999 70.059001) (width 0.35) (layer F.Cu) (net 18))
 (segment (start 19.082 72.204) (end 19.082 70.58) (width 0.35) (layer F.Cu) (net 18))
 (segment (start 19.602999 70.059001) (end 21.416001 70.059001) (width 0.35) (layer F.Cu) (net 18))
 (segment (start 21.416001 70.059001) (end 22.053001 69.422001) (width 0.35) (layer F.Cu) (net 18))
 (segment (start 22.053001 69.422001) (end 22.053001 67.519001) (width 0.35) (layer F.Cu) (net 18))
 (segment (start 22.053001 67.519001) (end 21.677999 67.143999) (width 0.35) (layer F.Cu) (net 18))
 (segment (start 23.882 83.052003) (end 23.876002 83.058001) (width 0.35) (layer F.Cu) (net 9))
 (segment (start 23.882 84.068002) (end 23.876002 84.074) (width 0.35) (layer F.Cu) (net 9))
 (segment (start 23.882 80.704) (end 23.882 84.068002) (width 0.35) (layer F.Cu) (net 9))
 (segment (start 25.332 78.454) (end 27.381 78.454) (width 0.35) (layer F.Cu) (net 10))
 (via (at 17.526 82.55) (size 0.8) (drill 0.4) (layers F.Cu B.Cu) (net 3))
 (segment (start 18.282 81.794) (end 17.526 82.55) (width 0.35) (layer F.Cu) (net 3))
 (segment (start 18.282 80.704) (end 18.282 81.794) (width 0.35) (layer F.Cu) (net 3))
 (segment (start 34.544 82.042) (end 34.544 68.834) (width 0.35) (layer B.Cu) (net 3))
 (segment (start 33.782 82.804) (end 34.544 82.042) (width 0.35) (layer B.Cu) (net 3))
 (segment (start 28.956 82.804) (end 33.782 82.804) (width 0.35) (layer B.Cu) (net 3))
 (segment (start 18.288 85.598) (end 27.432 85.598) (width 0.35) (layer B.Cu) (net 3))
 (segment (start 17.526 84.836) (end 18.288 85.598) (width 0.35) (layer B.Cu) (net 3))
 (segment (start 27.432 85.598) (end 28.194 84.836) (width 0.35) (layer B.Cu) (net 3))
 (segment (start 28.194 84.836) (end 28.194 83.566) (width 0.35) (layer B.Cu) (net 3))
 (segment (start 17.526 82.55) (end 17.526 84.836) (width 0.35) (layer B.Cu) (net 3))
 (segment (start 28.194 83.566) (end 28.956 82.804) (width 0.35) (layer B.Cu) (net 3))
 (segment (start 34.544 68.834) (end 34.544 72.136) (width 0.35) (layer F.Cu) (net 3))
 (segment (start 19.082 84.328) (end 15.748 84.328) (width 0.35) (layer F.Cu) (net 30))
 (segment (start 19.082 82.753) (end 19.082 80.704) (width 0.35) (layer F.Cu) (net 25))
 (segment (start 46.918 84.51) (end 46.918 88.478) (width 0.35) (layer F.Cu) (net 28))
 (segment (start 46.918 80.518) (end 46.918 84.51) (width 0.35) (layer F.Cu) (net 28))
 (segment (start 22.33201 83.844714) (end 22.33201 81.90401) (width 0.35) (layer F.Cu) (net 28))
 (segment (start 28.702 85.09) (end 23.577296 85.09) (width 0.35) (layer F.Cu) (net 28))
 (segment (start 22.33201 81.90401) (end 22.282 81.854) (width 0.35) (layer F.Cu) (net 28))
 (segment (start 40.64 90.17) (end 39.878 89.408) (width 0.35) (layer F.Cu) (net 28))
 (segment (start 46.918 84.51) (end 46.846 84.582) (width 0.35) (layer F.Cu) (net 28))
 (segment (start 23.577296 85.09) (end 22.33201 83.844714) (width 0.35) (layer F.Cu) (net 28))
 (segment (start 44.958 84.582) (end 44.196 85.344) (width 0.35) (layer F.Cu) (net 28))
 (segment (start 30.528749 83.263251) (end 28.702 85.09) (width 0.35) (layer F.Cu) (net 28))
 (segment (start 46.846 84.582) (end 44.958 84.582) (width 0.35) (layer F.Cu) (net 28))
 (segment (start 44.196 85.344) (end 44.196 89.662) (width 0.35) (layer F.Cu) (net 28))
 (segment (start 44.196 89.662) (end 43.688 90.17) (width 0.35) (layer F.Cu) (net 28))
 (segment (start 22.282 81.854) (end 22.282 80.704) (width 0.35) (layer F.Cu) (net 28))
 (segment (start 43.688 90.17) (end 40.64 90.17) (width 0.35) (layer F.Cu) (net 28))
 (segment (start 39.878 85.09) (end 38.051251 83.263251) (width 0.35) (layer F.Cu) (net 28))
 (segment (start 38.051251 83.263251) (end 30.528749 83.263251) (width 0.35) (layer F.Cu) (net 28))
 (segment (start 39.878 89.408) (end 39.878 85.09) (width 0.35) (layer F.Cu) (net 28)))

